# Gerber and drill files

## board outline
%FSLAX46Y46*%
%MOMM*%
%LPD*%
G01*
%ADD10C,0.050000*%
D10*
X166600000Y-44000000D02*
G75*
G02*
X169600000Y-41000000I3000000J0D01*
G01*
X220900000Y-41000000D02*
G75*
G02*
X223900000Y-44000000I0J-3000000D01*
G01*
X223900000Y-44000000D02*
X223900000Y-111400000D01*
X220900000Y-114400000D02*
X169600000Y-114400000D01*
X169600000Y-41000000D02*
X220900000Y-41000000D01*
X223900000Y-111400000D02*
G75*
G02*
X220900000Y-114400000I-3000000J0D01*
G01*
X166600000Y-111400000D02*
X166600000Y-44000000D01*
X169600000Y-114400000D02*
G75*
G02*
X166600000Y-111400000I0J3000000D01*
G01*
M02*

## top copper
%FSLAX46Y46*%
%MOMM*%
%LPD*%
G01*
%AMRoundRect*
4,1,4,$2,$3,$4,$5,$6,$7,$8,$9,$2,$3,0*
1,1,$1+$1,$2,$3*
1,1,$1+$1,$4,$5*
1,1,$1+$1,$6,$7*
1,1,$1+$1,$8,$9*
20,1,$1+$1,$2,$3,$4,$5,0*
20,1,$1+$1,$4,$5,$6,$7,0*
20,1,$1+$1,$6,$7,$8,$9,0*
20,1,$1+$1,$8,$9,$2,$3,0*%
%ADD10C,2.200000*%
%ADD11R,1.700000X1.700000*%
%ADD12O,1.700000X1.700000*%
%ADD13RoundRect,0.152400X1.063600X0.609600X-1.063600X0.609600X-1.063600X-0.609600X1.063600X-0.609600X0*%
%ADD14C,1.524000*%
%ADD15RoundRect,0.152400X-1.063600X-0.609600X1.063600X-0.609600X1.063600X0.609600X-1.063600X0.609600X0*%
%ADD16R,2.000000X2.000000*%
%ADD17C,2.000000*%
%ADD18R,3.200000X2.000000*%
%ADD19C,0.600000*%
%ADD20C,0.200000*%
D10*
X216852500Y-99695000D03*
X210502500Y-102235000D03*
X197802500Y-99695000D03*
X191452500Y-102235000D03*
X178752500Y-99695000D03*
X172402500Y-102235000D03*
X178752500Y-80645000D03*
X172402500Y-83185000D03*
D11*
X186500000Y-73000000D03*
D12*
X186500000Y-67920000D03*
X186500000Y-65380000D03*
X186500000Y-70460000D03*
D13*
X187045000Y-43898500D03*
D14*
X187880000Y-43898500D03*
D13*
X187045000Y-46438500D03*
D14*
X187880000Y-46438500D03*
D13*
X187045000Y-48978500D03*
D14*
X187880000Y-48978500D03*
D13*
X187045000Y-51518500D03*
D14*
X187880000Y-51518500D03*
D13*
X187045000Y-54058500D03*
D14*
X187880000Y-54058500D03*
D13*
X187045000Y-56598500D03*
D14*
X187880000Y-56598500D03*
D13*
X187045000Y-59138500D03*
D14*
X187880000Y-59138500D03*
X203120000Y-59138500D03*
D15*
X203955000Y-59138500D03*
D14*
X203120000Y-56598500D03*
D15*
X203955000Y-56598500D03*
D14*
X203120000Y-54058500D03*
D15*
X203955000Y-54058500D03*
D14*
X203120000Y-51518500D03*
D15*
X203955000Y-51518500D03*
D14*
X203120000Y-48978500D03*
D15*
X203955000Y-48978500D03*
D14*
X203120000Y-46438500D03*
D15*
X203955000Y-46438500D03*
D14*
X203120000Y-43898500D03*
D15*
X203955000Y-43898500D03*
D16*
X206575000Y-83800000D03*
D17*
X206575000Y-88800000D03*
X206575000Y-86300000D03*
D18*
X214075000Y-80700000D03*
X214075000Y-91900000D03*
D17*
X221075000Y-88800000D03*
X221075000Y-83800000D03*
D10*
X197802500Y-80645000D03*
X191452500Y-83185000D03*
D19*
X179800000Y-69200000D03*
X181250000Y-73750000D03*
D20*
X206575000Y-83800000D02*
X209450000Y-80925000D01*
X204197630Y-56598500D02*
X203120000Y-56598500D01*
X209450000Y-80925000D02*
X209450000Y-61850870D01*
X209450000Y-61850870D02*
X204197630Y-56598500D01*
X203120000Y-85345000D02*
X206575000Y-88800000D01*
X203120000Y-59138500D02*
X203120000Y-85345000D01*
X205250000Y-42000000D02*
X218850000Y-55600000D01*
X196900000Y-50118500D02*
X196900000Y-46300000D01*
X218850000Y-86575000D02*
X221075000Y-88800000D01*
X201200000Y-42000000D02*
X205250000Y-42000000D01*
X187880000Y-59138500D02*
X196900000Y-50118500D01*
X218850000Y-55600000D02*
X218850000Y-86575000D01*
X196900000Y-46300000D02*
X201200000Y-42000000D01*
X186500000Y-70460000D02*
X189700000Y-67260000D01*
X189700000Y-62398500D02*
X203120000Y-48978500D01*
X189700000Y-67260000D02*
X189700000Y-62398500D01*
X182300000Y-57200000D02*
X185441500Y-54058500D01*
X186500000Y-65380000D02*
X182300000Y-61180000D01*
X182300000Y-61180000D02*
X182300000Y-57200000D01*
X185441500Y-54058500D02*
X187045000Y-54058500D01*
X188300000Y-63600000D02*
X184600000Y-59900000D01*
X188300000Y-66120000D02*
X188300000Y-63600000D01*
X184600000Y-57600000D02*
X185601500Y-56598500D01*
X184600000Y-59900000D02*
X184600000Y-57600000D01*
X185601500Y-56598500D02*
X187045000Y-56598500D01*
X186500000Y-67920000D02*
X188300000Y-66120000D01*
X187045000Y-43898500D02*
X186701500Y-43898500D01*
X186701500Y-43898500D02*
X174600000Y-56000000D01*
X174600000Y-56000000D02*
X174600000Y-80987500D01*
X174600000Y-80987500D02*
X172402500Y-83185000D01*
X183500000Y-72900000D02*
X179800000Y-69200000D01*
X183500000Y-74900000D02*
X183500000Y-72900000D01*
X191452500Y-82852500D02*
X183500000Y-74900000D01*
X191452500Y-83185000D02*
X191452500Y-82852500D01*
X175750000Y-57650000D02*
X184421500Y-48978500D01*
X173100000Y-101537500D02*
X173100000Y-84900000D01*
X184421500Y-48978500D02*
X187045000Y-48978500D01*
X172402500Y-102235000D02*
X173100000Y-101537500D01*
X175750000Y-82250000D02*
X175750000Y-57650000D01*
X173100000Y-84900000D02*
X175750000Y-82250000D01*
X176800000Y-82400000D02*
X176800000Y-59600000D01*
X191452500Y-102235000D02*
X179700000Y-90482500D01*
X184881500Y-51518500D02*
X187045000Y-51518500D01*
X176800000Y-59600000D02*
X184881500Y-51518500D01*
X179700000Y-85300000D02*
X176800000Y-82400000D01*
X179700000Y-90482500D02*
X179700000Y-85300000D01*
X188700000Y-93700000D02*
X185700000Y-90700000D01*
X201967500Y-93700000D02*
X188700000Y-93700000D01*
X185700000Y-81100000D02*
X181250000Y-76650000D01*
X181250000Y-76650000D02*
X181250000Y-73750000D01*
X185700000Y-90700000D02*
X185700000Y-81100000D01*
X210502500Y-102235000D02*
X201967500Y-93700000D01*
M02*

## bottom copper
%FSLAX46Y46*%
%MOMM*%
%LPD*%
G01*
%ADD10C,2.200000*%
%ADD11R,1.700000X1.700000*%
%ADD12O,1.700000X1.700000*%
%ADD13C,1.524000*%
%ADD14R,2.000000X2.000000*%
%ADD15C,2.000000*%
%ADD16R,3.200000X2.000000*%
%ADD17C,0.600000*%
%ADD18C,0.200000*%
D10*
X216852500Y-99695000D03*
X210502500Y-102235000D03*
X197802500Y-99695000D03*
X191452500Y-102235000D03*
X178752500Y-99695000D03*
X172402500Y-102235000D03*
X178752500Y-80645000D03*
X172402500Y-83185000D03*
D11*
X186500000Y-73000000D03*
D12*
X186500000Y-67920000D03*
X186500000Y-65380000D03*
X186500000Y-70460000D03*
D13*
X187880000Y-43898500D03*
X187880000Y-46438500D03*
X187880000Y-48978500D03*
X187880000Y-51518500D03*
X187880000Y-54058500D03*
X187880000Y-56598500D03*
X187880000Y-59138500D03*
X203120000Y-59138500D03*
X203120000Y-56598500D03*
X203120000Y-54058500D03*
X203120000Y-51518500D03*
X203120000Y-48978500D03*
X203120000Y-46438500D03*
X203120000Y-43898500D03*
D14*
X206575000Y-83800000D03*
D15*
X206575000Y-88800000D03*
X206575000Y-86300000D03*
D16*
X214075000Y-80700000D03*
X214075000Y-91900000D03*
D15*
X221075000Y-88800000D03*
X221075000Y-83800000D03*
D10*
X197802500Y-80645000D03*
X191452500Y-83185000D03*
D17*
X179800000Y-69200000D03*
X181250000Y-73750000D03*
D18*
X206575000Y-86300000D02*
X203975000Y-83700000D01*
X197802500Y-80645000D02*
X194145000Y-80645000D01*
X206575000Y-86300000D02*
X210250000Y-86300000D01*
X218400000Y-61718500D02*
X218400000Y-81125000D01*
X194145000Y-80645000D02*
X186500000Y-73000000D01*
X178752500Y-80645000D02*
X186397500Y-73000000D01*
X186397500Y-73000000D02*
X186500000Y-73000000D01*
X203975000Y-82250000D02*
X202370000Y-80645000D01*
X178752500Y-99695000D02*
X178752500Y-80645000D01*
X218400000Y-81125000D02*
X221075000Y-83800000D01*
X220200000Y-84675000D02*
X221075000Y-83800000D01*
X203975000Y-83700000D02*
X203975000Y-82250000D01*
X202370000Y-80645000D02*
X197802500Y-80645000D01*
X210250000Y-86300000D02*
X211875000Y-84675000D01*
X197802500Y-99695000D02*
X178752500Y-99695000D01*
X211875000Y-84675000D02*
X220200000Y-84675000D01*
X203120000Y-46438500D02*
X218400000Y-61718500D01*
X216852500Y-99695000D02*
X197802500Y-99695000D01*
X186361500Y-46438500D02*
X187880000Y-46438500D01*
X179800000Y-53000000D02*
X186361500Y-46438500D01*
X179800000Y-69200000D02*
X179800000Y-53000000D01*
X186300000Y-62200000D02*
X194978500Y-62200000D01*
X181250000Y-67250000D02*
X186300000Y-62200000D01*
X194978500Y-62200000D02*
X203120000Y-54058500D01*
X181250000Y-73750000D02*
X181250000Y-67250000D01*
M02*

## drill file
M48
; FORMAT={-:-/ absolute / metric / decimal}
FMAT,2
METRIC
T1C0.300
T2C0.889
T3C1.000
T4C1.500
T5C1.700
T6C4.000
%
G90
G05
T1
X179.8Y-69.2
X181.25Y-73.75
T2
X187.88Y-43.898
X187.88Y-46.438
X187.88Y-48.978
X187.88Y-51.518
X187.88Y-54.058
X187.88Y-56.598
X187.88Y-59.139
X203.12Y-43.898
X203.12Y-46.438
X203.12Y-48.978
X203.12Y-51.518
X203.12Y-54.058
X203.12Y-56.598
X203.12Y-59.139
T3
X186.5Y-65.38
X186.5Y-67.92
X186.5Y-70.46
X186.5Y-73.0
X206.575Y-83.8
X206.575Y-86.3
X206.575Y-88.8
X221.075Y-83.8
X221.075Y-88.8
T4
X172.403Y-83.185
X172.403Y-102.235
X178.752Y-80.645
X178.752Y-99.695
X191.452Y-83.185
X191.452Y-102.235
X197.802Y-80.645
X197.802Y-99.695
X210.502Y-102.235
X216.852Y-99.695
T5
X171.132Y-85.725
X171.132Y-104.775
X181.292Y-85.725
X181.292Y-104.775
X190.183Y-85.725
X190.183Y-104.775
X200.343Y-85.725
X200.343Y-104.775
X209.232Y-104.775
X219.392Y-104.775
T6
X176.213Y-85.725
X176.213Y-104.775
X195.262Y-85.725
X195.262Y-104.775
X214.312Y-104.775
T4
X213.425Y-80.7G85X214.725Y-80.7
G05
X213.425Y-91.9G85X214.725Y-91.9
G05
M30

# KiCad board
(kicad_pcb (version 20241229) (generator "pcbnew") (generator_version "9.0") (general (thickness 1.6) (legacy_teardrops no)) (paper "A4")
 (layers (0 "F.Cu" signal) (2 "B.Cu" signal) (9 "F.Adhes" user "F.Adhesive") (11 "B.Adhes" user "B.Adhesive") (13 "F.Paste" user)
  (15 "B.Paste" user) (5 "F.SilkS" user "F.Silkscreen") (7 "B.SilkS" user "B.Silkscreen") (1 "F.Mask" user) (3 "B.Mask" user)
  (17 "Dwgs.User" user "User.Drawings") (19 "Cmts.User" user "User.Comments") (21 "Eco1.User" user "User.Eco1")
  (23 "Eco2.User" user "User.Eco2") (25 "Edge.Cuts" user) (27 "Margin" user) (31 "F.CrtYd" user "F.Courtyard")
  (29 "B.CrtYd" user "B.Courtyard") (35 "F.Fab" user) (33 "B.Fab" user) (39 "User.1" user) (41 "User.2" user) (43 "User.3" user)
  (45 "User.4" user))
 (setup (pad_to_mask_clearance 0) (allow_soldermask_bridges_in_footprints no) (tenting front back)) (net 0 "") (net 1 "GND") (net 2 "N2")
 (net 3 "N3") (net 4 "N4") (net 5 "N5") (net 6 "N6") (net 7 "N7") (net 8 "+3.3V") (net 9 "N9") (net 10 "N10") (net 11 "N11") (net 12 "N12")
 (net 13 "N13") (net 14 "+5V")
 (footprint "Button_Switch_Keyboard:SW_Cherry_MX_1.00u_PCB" (layer "F.Cu") (at 216.8525 99.695)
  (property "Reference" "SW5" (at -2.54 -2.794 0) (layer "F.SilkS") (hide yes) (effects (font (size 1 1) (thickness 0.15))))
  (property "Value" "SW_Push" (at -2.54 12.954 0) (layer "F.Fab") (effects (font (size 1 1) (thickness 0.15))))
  (pad "" np_thru_hole circle (at -7.62 5.08) (size 1.7 1.7) (drill 1.7) (layers "*.Cu" "*.Mask"))
  (pad "" np_thru_hole circle (at -2.54 5.08) (size 4 4) (drill 4) (layers "*.Cu" "*.Mask"))
  (pad "" np_thru_hole circle (at 2.54 5.08) (size 1.7 1.7) (drill 1.7) (layers "*.Cu" "*.Mask"))
  (pad "1" thru_hole circle (at 0 0) (size 2.2 2.2) (drill 1.5) (layers "*.Cu" "*.Mask") (remove_unused_layers no) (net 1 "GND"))
  (pad "2" thru_hole circle (at -6.35 2.54) (size 2.2 2.2) (drill 1.5) (layers "*.Cu" "*.Mask") (remove_unused_layers no) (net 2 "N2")))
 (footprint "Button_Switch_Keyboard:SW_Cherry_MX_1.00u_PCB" (layer "F.Cu") (at 197.8025 99.695)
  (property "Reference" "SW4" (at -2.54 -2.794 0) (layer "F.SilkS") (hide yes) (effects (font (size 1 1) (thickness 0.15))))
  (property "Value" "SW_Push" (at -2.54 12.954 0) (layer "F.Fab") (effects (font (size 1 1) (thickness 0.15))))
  (pad "" np_thru_hole circle (at -7.62 5.08) (size 1.7 1.7) (drill 1.7) (layers "*.Cu" "*.Mask"))
  (pad "" np_thru_hole circle (at -2.54 5.08) (size 4 4) (drill 4) (layers "*.Cu" "*.Mask"))
  (pad "" np_thru_hole circle (at 2.54 5.08) (size 1.7 1.7) (drill 1.7) (layers "*.Cu" "*.Mask"))
  (pad "1" thru_hole circle (at 0 0) (size 2.2 2.2) (drill 1.5) (layers "*.Cu" "*.Mask") (remove_unused_layers no) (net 1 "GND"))
  (pad "2" thru_hole circle (at -6.35 2.54) (size 2.2 2.2) (drill 1.5) (layers "*.Cu" "*.Mask") (remove_unused_layers no) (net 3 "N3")))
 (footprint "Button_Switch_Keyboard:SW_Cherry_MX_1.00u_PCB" (layer "F.Cu") (at 178.7525 99.695)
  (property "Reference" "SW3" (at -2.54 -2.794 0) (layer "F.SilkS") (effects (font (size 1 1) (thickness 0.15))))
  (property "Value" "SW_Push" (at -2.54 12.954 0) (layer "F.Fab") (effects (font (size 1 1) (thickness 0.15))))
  (pad "" np_thru_hole circle (at -7.62 5.08) (size 1.7 1.7) (drill 1.7) (layers "*.Cu" "*.Mask"))
  (pad "" np_thru_hole circle (at -2.54 5.08) (size 4 4) (drill 4) (layers "*.Cu" "*.Mask"))
  (pad "" np_thru_hole circle (at 2.54 5.08) (size 1.7 1.7) (drill 1.7) (layers "*.Cu" "*.Mask"))
  (pad "1" thru_hole circle (at 0 0) (size 2.2 2.2) (drill 1.5) (layers "*.Cu" "*.Mask") (remove_unused_layers no) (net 1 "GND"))
  (pad "2" thru_hole circle (at -6.35 2.54) (size 2.2 2.2) (drill 1.5) (layers "*.Cu" "*.Mask") (remove_unused_layers no) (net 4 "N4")))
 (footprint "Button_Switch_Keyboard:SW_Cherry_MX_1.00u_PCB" (layer "F.Cu") (at 178.7525 80.645)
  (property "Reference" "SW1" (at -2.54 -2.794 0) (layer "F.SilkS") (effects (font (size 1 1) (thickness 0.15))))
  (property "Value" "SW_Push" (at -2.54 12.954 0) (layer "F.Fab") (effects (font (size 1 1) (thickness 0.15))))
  (pad "" np_thru_hole circle (at -7.62 5.08) (size 1.7 1.7) (drill 1.7) (layers "*.Cu" "*.Mask"))
  (pad "" np_thru_hole circle (at -2.54 5.08) (size 4 4) (drill 4) (layers "*.Cu" "*.Mask"))
  (pad "" np_thru_hole circle (at 2.54 5.08) (size 1.7 1.7) (drill 1.7) (layers "*.Cu" "*.Mask"))
  (pad "1" thru_hole circle (at 0 0) (size 2.2 2.2) (drill 1.5) (layers "*.Cu" "*.Mask") (remove_unused_layers no) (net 1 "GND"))
  (pad "2" thru_hole circle (at -6.35 2.54) (size 2.2 2.2) (drill 1.5) (layers "*.Cu" "*.Mask") (remove_unused_layers no) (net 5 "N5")))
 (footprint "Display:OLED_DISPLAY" (layer "F.Cu") (at 204.2 69.23)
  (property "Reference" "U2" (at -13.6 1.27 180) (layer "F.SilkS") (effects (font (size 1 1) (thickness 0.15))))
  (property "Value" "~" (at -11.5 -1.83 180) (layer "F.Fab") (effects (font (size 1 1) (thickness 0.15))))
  (pad "GND" thru_hole rect (at -17.7 3.77 180) (size 1.7 1.7) (drill 1) (layers "*.Cu" "*.Mask") (remove_unused_layers no) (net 1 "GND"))
  (pad "SCL" thru_hole oval (at -17.7 -1.31 180) (size 1.7 1.7) (drill 1) (layers "*.Cu" "*.Mask") (remove_unused_layers no) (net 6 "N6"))
  (pad "SDA" thru_hole oval (at -17.7 -3.85 180) (size 1.7 1.7) (drill 1) (layers "*.Cu" "*.Mask") (remove_unused_layers no) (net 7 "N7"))
  (pad "VCC" thru_hole oval (at -17.7 1.23 180) (size 1.7 1.7) (drill 1) (layers "*.Cu" "*.Mask") (remove_unused_layers no) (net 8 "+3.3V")))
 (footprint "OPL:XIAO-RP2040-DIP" (layer "F.Cu") (at 195.5 51.5185)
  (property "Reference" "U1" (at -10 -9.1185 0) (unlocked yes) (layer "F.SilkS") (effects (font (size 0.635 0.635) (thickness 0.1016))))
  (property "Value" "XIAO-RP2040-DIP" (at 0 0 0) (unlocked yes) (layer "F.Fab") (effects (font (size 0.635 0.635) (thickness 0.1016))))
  (pad "1" smd roundrect (at -8.455 -7.62 180) (size 2.432 1.524) (layers "F.Cu" "F.Mask") (roundrect_rratio 0.1) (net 5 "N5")
   (thermal_bridge_angle 45))
  (pad "1" thru_hole circle (at -7.62 -7.62 180) (size 1.524 1.524) (drill 0.889) (layers "*.Cu" "*.Mask") (remove_unused_layers no)
   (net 5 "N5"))
  (pad "2" smd roundrect (at -8.455 -5.08 180) (size 2.432 1.524) (layers "F.Cu" "F.Mask") (roundrect_rratio 0.1) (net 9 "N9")
   (thermal_bridge_angle 45))
  (pad "2" thru_hole circle (at -7.62 -5.08 180) (size 1.524 1.524) (drill 0.889) (layers "*.Cu" "*.Mask") (remove_unused_layers no)
   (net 9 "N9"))
  (pad "3" smd roundrect (at -8.455 -2.54 180) (size 2.432 1.524) (layers "F.Cu" "F.Mask") (roundrect_rratio 0.1) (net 4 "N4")
   (thermal_bridge_angle 45))
  (pad "3" thru_hole circle (at -7.62 -2.54 180) (size 1.524 1.524) (drill 0.889) (layers "*.Cu" "*.Mask") (remove_unused_layers no)
   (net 4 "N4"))
  (pad "4" smd roundrect (at -8.455 0 180) (size 2.432 1.524) (layers "F.Cu" "F.Mask") (roundrect_rratio 0.1) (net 3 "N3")
   (thermal_bridge_angle 45))
  (pad "4" thru_hole circle (at -7.62 0 180) (size 1.524 1.524) (drill 0.889) (layers "*.Cu" "*.Mask") (remove_unused_layers no)
   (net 3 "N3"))
  (pad "5" smd roundrect (at -8.455 2.54 180) (size 2.432 1.524) (layers "F.Cu" "F.Mask") (roundrect_rratio 0.1) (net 7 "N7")
   (thermal_bridge_angle 45))
  (pad "5" thru_hole circle (at -7.62 2.54 180) (size 1.524 1.524) (drill 0.889) (layers "*.Cu" "*.Mask") (remove_unused_layers no)
   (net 7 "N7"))
  (pad "6" smd roundrect (at -8.455 5.08 180) (size 2.432 1.524) (layers "F.Cu" "F.Mask") (roundrect_rratio 0.1) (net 6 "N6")
   (thermal_bridge_angle 45))
  (pad "6" thru_hole circle (at -7.62 5.08 180) (size 1.524 1.524) (drill 0.889) (layers "*.Cu" "*.Mask") (remove_unused_layers no)
   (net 6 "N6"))
  (pad "7" smd roundrect (at -8.455 7.62 180) (size 2.432 1.524) (layers "F.Cu" "F.Mask") (roundrect_rratio 0.1) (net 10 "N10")
   (thermal_bridge_angle 45))
  (pad "7" thru_hole circle (at -7.62 7.62 180) (size 1.524 1.524) (drill 0.889) (layers "*.Cu" "*.Mask") (remove_unused_layers no)
   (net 10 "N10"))
  (pad "8" thru_hole circle (at 7.62 7.62) (size 1.524 1.524) (drill 0.889) (layers "*.Cu" "*.Mask") (remove_unused_layers no)
   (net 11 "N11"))
  (pad "8" smd roundrect (at 8.455 7.62) (size 2.432 1.524) (layers "F.Cu" "F.Mask") (roundrect_rratio 0.1) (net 11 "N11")
   (thermal_bridge_angle 45))
  (pad "9" thru_hole circle (at 7.62 5.08) (size 1.524 1.524) (drill 0.889) (layers "*.Cu" "*.Mask") (remove_unused_layers no)
   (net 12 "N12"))
  (pad "9" smd roundrect (at 8.455 5.08) (size 2.432 1.524) (layers "F.Cu" "F.Mask") (roundrect_rratio 0.1) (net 12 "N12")
   (thermal_bridge_angle 45))
  (pad "10" thru_hole circle (at 7.62 2.54) (size 1.524 1.524) (drill 0.889) (layers "*.Cu" "*.Mask") (remove_unused_layers no) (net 2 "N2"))
  (pad "10" smd roundrect (at 8.455 2.54) (size 2.432 1.524) (layers "F.Cu" "F.Mask") (roundrect_rratio 0.1) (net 2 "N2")
   (thermal_bridge_angle 45))
  (pad "11" thru_hole circle (at 7.62 0) (size 1.524 1.524) (drill 0.889) (layers "*.Cu" "*.Mask") (remove_unused_layers no) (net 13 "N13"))
  (pad "11" smd roundrect (at 8.455 0) (size 2.432 1.524) (layers "F.Cu" "F.Mask") (roundrect_rratio 0.1) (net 13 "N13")
   (thermal_bridge_angle 45))
  (pad "12" thru_hole circle (at 7.62 -2.54) (size 1.524 1.524) (drill 0.889) (layers "*.Cu" "*.Mask") (remove_unused_layers no)
   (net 8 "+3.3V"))
  (pad "12" smd roundrect (at 8.455 -2.54) (size 2.432 1.524) (layers "F.Cu" "F.Mask") (roundrect_rratio 0.1) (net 8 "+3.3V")
   (thermal_bridge_angle 45))
  (pad "13" thru_hole circle (at 7.62 -5.08) (size 1.524 1.524) (drill 0.889) (layers "*.Cu" "*.Mask") (remove_unused_layers no)
   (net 1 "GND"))
  (pad "13" smd roundrect (at 8.455 -5.08) (size 2.432 1.524) (layers "F.Cu" "F.Mask") (roundrect_rratio 0.1) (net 1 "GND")
   (thermal_bridge_angle 45))
  (pad "14" thru_hole circle (at 7.62 -7.62) (size 1.524 1.524) (drill 0.889) (layers "*.Cu" "*.Mask") (remove_unused_layers no)
   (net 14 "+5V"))
  (pad "14" smd roundrect (at 8.455 -7.62) (size 2.432 1.524) (layers "F.Cu" "F.Mask") (roundrect_rratio 0.1) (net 14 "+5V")
   (thermal_bridge_angle 45)))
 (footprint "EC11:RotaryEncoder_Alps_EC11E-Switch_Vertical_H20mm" (layer "F.Cu") (at 206.575 83.8)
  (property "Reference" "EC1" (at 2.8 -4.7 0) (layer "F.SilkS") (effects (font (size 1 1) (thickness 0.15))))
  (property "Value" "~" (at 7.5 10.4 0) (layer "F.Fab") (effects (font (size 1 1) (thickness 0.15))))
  (pad "A" thru_hole rect (at 0 0) (size 2 2) (drill 1) (layers "*.Cu" "*.Mask") (remove_unused_layers no) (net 12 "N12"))
  (pad "B" thru_hole circle (at 0 5) (size 2 2) (drill 1) (layers "*.Cu" "*.Mask") (remove_unused_layers no) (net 11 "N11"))
  (pad "C" thru_hole circle (at 0 2.5) (size 2 2) (drill 1) (layers "*.Cu" "*.Mask") (remove_unused_layers no) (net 1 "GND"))
  (pad "MP" thru_hole rect (at 7.5 -3.1) (size 3.2 2) (drill oval 2.8 1.5) (layers "*.Cu" "*.Mask") (remove_unused_layers no))
  (pad "MP" thru_hole rect (at 7.5 8.1) (size 3.2 2) (drill oval 2.8 1.5) (layers "*.Cu" "*.Mask") (remove_unused_layers no))
  (pad "S1" thru_hole circle (at 14.5 5) (size 2 2) (drill 1) (layers "*.Cu" "*.Mask") (remove_unused_layers no) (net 10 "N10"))
  (pad "S2" thru_hole circle (at 14.5 0) (size 2 2) (drill 1) (layers "*.Cu" "*.Mask") (remove_unused_layers no) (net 1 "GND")))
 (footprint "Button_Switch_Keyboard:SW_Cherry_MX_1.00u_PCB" (layer "F.Cu") (at 197.8025 80.645)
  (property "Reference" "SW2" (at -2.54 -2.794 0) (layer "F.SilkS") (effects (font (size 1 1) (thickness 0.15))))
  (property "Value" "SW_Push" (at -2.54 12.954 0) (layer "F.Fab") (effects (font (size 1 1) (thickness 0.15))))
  (pad "" np_thru_hole circle (at -7.62 5.08) (size 1.7 1.7) (drill 1.7) (layers "*.Cu" "*.Mask"))
  (pad "" np_thru_hole circle (at -2.54 5.08) (size 4 4) (drill 4) (layers "*.Cu" "*.Mask"))
  (pad "" np_thru_hole circle (at 2.54 5.08) (size 1.7 1.7) (drill 1.7) (layers "*.Cu" "*.Mask"))
  (pad "1" thru_hole circle (at 0 0) (size 2.2 2.2) (drill 1.5) (layers "*.Cu" "*.Mask") (remove_unused_layers no) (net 1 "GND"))
  (pad "2" thru_hole circle (at -6.35 2.54) (size 2.2 2.2) (drill 1.5) (layers "*.Cu" "*.Mask") (remove_unused_layers no) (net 9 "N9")))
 (gr_arc (start 166.6 44) (mid 167.47868 41.87868) (end 169.6 41) (stroke (width 0.05) (type default)) (layer "Edge.Cuts"))
 (gr_arc (start 220.9 41) (mid 223.02132 41.87868) (end 223.9 44) (stroke (width 0.05) (type default)) (layer "Edge.Cuts"))
 (gr_line (start 223.9 44) (end 223.9 111.4) (stroke (width 0.05) (type default)) (layer "Edge.Cuts"))
 (gr_line (start 220.9 114.4) (end 169.6 114.4) (stroke (width 0.05) (type default)) (layer "Edge.Cuts"))
 (gr_line (start 169.6 41) (end 220.9 41) (stroke (width 0.05) (type default)) (layer "Edge.Cuts"))
 (gr_arc (start 223.9 111.4) (mid 223.02132 113.52132) (end 220.9 114.4) (stroke (width 0.05) (type default)) (layer "Edge.Cuts"))
 (gr_line (start 166.6 111.4) (end 166.6 44) (stroke (width 0.05) (type default)) (layer "Edge.Cuts"))
 (gr_arc (start 169.6 114.4) (mid 167.47868 113.52132) (end 166.6 111.4) (stroke (width 0.05) (type default)) (layer "Edge.Cuts"))
 (segment (start 206.575 86.3) (end 203.975 83.7) (width 0.2) (layer "B.Cu") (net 1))
 (segment (start 197.8025 80.645) (end 194.145 80.645) (width 0.2) (layer "B.Cu") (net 1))
 (segment (start 206.575 86.3) (end 210.25 86.3) (width 0.2) (layer "B.Cu") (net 1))
 (segment (start 218.4 61.7185) (end 218.4 81.125) (width 0.2) (layer "B.Cu") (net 1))
 (segment (start 194.145 80.645) (end 186.5 73) (width 0.2) (layer "B.Cu") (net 1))
 (segment (start 178.7525 80.645) (end 186.3975 73) (width 0.2) (layer "B.Cu") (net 1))
 (segment (start 186.3975 73) (end 186.5 73) (width 0.2) (layer "B.Cu") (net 1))
 (segment (start 203.975 82.25) (end 202.37 80.645) (width 0.2) (layer "B.Cu") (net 1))
 (segment (start 178.7525 99.695) (end 178.7525 80.645) (width 0.2) (layer "B.Cu") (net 1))
 (segment (start 218.4 81.125) (end 221.075 83.8) (width 0.2) (layer "B.Cu") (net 1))
 (segment (start 220.2 84.675) (end 221.075 83.8) (width 0.2) (layer "B.Cu") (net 1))
 (segment (start 203.975 83.7) (end 203.975 82.25) (width 0.2) (layer "B.Cu") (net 1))
 (segment (start 202.37 80.645) (end 197.8025 80.645) (width 0.2) (layer "B.Cu") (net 1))
 (segment (start 210.25 86.3) (end 211.875 84.675) (width 0.2) (layer "B.Cu") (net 1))
 (segment (start 197.8025 99.695) (end 178.7525 99.695) (width 0.2) (layer "B.Cu") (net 1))
 (segment (start 211.875 84.675) (end 220.2 84.675) (width 0.2) (layer "B.Cu") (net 1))
 (segment (start 203.12 46.4385) (end 218.4 61.7185) (width 0.2) (layer "B.Cu") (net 1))
 (segment (start 216.8525 99.695) (end 197.8025 99.695) (width 0.2) (layer "B.Cu") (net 1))
 (segment (start 206.575 83.8) (end 209.45 80.925) (width 0.2) (layer "F.Cu") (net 12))
 (segment (start 204.19763 56.5985) (end 203.12 56.5985) (width 0.2) (layer "F.Cu") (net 12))
 (segment (start 209.45 80.925) (end 209.45 61.85087) (width 0.2) (layer "F.Cu") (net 12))
 (segment (start 209.45 61.85087) (end 204.19763 56.5985) (width 0.2) (layer "F.Cu") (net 12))
 (segment (start 203.12 85.345) (end 206.575 88.8) (width 0.2) (layer "F.Cu") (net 11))
 (segment (start 203.12 59.1385) (end 203.12 85.345) (width 0.2) (layer "F.Cu") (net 11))
 (segment (start 205.25 42) (end 218.85 55.6) (width 0.2) (layer "F.Cu") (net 10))
 (segment (start 196.9 50.1185) (end 196.9 46.3) (width 0.2) (layer "F.Cu") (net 10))
 (segment (start 218.85 86.575) (end 221.075 88.8) (width 0.2) (layer "F.Cu") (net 10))
 (segment (start 201.2 42) (end 205.25 42) (width 0.2) (layer "F.Cu") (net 10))
 (segment (start 187.88 59.1385) (end 196.9 50.1185) (width 0.2) (layer "F.Cu") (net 10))
 (segment (start 218.85 55.6) (end 218.85 86.575) (width 0.2) (layer "F.Cu") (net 10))
 (segment (start 196.9 46.3) (end 201.2 42) (width 0.2) (layer "F.Cu") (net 10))
 (segment (start 186.5 70.46) (end 189.7 67.26) (width 0.2) (layer "F.Cu") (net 8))
 (segment (start 189.7 62.3985) (end 203.12 48.9785) (width 0.2) (layer "F.Cu") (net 8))
 (segment (start 189.7 67.26) (end 189.7 62.3985) (width 0.2) (layer "F.Cu") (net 8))
 (segment (start 182.3 57.2) (end 185.4415 54.0585) (width 0.2) (layer "F.Cu") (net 7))
 (segment (start 186.5 65.38) (end 182.3 61.18) (width 0.2) (layer "F.Cu") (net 7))
 (segment (start 182.3 61.18) (end 182.3 57.2) (width 0.2) (layer "F.Cu") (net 7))
 (segment (start 185.4415 54.0585) (end 187.045 54.0585) (width 0.2) (layer "F.Cu") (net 7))
 (segment (start 188.3 63.6) (end 184.6 59.9) (width 0.2) (layer "F.Cu") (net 6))
 (segment (start 188.3 66.12) (end 188.3 63.6) (width 0.2) (layer "F.Cu") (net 6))
 (segment (start 184.6 57.6) (end 185.6015 56.5985) (width 0.2) (layer "F.Cu") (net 6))
 (segment (start 184.6 59.9) (end 184.6 57.6) (width 0.2) (layer "F.Cu") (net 6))
 (segment (start 185.6015 56.5985) (end 187.045 56.5985) (width 0.2) (layer "F.Cu") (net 6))
 (segment (start 186.5 67.92) (end 188.3 66.12) (width 0.2) (layer "F.Cu") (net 6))
 (segment (start 187.045 43.8985) (end 186.7015 43.8985) (width 0.2) (layer "F.Cu") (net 5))
 (segment (start 186.7015 43.8985) (end 174.6 56) (width 0.2) (layer "F.Cu") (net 5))
 (segment (start 174.6 56) (end 174.6 80.9875) (width 0.2) (layer "F.Cu") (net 5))
 (segment (start 174.6 80.9875) (end 172.4025 83.185) (width 0.2) (layer "F.Cu") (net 5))
 (segment (start 183.5 72.9) (end 179.8 69.2) (width 0.2) (layer "F.Cu") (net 9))
 (segment (start 183.5 74.9) (end 183.5 72.9) (width 0.2) (layer "F.Cu") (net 9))
 (segment (start 191.4525 82.8525) (end 183.5 74.9) (width 0.2) (layer "F.Cu") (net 9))
 (segment (start 191.4525 83.185) (end 191.4525 82.8525) (width 0.2) (layer "F.Cu") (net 9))
 (via (at 179.8 69.2) (size 0.6) (drill 0.3) (layers "F.Cu" "B.Cu") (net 9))
 (segment (start 186.3615 46.4385) (end 187.88 46.4385) (width 0.2) (layer "B.Cu") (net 9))
 (segment (start 179.8 53) (end 186.3615 46.4385) (width 0.2) (layer "B.Cu") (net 9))
 (segment (start 179.8 69.2) (end 179.8 53) (width 0.2) (layer "B.Cu") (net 9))
 (segment (start 175.75 57.65) (end 184.4215 48.9785) (width 0.2) (layer "F.Cu") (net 4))
 (segment (start 173.1 101.5375) (end 173.1 84.9) (width 0.2) (layer "F.Cu") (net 4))
 (segment (start 184.4215 48.9785) (end 187.045 48.9785) (width 0.2) (layer "F.Cu") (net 4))
 (segment (start 172.4025 102.235) (end 173.1 101.5375) (width 0.2) (layer "F.Cu") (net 4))
 (segment (start 175.75 82.25) (end 175.75 57.65) (width 0.2) (layer "F.Cu") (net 4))
 (segment (start 173.1 84.9) (end 175.75 82.25) (width 0.2) (layer "F.Cu") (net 4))
 (segment (start 176.8 82.4) (end 176.8 59.6) (width 0.2) (layer "F.Cu") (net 3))
 (segment (start 191.4525 102.235) (end 179.7 90.4825) (width 0.2) (layer "F.Cu") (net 3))
 (segment (start 184.8815 51.5185) (end 187.045 51.5185) (width 0.2) (layer "F.Cu") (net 3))
 (segment (start 176.8 59.6) (end 184.8815 51.5185) (width 0.2) (layer "F.Cu") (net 3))
 (segment (start 179.7 85.3) (end 176.8 82.4) (width 0.2) (layer "F.Cu") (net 3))
 (segment (start 179.7 90.4825) (end 179.7 85.3) (width 0.2) (layer "F.Cu") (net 3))
 (segment (start 188.7 93.7) (end 185.7 90.7) (width 0.2) (layer "F.Cu") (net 2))
 (segment (start 201.9675 93.7) (end 188.7 93.7) (width 0.2) (layer "F.Cu") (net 2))
 (segment (start 185.7 81.1) (end 181.25 76.65) (width 0.2) (layer "F.Cu") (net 2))
 (segment (start 181.25 76.65) (end 181.25 73.75) (width 0.2) (layer "F.Cu") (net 2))
 (segment (start 185.7 90.7) (end 185.7 81.1) (width 0.2) (layer "F.Cu") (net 2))
 (segment (start 210.5025 102.235) (end 201.9675 93.7) (width 0.2) (layer "F.Cu") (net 2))
 (via (at 181.25 73.75) (size 0.6) (drill 0.3) (layers "F.Cu" "B.Cu") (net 2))
 (segment (start 186.3 62.2) (end 194.9785 62.2) (width 0.2) (layer "B.Cu") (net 2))
 (segment (start 181.25 67.25) (end 186.3 62.2) (width 0.2) (layer "B.Cu") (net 2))
 (segment (start 194.9785 62.2) (end 203.12 54.0585) (width 0.2) (layer "B.Cu") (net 2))
 (segment (start 181.25 73.75) (end 181.25 67.25) (width 0.2) (layer "B.Cu") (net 2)))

